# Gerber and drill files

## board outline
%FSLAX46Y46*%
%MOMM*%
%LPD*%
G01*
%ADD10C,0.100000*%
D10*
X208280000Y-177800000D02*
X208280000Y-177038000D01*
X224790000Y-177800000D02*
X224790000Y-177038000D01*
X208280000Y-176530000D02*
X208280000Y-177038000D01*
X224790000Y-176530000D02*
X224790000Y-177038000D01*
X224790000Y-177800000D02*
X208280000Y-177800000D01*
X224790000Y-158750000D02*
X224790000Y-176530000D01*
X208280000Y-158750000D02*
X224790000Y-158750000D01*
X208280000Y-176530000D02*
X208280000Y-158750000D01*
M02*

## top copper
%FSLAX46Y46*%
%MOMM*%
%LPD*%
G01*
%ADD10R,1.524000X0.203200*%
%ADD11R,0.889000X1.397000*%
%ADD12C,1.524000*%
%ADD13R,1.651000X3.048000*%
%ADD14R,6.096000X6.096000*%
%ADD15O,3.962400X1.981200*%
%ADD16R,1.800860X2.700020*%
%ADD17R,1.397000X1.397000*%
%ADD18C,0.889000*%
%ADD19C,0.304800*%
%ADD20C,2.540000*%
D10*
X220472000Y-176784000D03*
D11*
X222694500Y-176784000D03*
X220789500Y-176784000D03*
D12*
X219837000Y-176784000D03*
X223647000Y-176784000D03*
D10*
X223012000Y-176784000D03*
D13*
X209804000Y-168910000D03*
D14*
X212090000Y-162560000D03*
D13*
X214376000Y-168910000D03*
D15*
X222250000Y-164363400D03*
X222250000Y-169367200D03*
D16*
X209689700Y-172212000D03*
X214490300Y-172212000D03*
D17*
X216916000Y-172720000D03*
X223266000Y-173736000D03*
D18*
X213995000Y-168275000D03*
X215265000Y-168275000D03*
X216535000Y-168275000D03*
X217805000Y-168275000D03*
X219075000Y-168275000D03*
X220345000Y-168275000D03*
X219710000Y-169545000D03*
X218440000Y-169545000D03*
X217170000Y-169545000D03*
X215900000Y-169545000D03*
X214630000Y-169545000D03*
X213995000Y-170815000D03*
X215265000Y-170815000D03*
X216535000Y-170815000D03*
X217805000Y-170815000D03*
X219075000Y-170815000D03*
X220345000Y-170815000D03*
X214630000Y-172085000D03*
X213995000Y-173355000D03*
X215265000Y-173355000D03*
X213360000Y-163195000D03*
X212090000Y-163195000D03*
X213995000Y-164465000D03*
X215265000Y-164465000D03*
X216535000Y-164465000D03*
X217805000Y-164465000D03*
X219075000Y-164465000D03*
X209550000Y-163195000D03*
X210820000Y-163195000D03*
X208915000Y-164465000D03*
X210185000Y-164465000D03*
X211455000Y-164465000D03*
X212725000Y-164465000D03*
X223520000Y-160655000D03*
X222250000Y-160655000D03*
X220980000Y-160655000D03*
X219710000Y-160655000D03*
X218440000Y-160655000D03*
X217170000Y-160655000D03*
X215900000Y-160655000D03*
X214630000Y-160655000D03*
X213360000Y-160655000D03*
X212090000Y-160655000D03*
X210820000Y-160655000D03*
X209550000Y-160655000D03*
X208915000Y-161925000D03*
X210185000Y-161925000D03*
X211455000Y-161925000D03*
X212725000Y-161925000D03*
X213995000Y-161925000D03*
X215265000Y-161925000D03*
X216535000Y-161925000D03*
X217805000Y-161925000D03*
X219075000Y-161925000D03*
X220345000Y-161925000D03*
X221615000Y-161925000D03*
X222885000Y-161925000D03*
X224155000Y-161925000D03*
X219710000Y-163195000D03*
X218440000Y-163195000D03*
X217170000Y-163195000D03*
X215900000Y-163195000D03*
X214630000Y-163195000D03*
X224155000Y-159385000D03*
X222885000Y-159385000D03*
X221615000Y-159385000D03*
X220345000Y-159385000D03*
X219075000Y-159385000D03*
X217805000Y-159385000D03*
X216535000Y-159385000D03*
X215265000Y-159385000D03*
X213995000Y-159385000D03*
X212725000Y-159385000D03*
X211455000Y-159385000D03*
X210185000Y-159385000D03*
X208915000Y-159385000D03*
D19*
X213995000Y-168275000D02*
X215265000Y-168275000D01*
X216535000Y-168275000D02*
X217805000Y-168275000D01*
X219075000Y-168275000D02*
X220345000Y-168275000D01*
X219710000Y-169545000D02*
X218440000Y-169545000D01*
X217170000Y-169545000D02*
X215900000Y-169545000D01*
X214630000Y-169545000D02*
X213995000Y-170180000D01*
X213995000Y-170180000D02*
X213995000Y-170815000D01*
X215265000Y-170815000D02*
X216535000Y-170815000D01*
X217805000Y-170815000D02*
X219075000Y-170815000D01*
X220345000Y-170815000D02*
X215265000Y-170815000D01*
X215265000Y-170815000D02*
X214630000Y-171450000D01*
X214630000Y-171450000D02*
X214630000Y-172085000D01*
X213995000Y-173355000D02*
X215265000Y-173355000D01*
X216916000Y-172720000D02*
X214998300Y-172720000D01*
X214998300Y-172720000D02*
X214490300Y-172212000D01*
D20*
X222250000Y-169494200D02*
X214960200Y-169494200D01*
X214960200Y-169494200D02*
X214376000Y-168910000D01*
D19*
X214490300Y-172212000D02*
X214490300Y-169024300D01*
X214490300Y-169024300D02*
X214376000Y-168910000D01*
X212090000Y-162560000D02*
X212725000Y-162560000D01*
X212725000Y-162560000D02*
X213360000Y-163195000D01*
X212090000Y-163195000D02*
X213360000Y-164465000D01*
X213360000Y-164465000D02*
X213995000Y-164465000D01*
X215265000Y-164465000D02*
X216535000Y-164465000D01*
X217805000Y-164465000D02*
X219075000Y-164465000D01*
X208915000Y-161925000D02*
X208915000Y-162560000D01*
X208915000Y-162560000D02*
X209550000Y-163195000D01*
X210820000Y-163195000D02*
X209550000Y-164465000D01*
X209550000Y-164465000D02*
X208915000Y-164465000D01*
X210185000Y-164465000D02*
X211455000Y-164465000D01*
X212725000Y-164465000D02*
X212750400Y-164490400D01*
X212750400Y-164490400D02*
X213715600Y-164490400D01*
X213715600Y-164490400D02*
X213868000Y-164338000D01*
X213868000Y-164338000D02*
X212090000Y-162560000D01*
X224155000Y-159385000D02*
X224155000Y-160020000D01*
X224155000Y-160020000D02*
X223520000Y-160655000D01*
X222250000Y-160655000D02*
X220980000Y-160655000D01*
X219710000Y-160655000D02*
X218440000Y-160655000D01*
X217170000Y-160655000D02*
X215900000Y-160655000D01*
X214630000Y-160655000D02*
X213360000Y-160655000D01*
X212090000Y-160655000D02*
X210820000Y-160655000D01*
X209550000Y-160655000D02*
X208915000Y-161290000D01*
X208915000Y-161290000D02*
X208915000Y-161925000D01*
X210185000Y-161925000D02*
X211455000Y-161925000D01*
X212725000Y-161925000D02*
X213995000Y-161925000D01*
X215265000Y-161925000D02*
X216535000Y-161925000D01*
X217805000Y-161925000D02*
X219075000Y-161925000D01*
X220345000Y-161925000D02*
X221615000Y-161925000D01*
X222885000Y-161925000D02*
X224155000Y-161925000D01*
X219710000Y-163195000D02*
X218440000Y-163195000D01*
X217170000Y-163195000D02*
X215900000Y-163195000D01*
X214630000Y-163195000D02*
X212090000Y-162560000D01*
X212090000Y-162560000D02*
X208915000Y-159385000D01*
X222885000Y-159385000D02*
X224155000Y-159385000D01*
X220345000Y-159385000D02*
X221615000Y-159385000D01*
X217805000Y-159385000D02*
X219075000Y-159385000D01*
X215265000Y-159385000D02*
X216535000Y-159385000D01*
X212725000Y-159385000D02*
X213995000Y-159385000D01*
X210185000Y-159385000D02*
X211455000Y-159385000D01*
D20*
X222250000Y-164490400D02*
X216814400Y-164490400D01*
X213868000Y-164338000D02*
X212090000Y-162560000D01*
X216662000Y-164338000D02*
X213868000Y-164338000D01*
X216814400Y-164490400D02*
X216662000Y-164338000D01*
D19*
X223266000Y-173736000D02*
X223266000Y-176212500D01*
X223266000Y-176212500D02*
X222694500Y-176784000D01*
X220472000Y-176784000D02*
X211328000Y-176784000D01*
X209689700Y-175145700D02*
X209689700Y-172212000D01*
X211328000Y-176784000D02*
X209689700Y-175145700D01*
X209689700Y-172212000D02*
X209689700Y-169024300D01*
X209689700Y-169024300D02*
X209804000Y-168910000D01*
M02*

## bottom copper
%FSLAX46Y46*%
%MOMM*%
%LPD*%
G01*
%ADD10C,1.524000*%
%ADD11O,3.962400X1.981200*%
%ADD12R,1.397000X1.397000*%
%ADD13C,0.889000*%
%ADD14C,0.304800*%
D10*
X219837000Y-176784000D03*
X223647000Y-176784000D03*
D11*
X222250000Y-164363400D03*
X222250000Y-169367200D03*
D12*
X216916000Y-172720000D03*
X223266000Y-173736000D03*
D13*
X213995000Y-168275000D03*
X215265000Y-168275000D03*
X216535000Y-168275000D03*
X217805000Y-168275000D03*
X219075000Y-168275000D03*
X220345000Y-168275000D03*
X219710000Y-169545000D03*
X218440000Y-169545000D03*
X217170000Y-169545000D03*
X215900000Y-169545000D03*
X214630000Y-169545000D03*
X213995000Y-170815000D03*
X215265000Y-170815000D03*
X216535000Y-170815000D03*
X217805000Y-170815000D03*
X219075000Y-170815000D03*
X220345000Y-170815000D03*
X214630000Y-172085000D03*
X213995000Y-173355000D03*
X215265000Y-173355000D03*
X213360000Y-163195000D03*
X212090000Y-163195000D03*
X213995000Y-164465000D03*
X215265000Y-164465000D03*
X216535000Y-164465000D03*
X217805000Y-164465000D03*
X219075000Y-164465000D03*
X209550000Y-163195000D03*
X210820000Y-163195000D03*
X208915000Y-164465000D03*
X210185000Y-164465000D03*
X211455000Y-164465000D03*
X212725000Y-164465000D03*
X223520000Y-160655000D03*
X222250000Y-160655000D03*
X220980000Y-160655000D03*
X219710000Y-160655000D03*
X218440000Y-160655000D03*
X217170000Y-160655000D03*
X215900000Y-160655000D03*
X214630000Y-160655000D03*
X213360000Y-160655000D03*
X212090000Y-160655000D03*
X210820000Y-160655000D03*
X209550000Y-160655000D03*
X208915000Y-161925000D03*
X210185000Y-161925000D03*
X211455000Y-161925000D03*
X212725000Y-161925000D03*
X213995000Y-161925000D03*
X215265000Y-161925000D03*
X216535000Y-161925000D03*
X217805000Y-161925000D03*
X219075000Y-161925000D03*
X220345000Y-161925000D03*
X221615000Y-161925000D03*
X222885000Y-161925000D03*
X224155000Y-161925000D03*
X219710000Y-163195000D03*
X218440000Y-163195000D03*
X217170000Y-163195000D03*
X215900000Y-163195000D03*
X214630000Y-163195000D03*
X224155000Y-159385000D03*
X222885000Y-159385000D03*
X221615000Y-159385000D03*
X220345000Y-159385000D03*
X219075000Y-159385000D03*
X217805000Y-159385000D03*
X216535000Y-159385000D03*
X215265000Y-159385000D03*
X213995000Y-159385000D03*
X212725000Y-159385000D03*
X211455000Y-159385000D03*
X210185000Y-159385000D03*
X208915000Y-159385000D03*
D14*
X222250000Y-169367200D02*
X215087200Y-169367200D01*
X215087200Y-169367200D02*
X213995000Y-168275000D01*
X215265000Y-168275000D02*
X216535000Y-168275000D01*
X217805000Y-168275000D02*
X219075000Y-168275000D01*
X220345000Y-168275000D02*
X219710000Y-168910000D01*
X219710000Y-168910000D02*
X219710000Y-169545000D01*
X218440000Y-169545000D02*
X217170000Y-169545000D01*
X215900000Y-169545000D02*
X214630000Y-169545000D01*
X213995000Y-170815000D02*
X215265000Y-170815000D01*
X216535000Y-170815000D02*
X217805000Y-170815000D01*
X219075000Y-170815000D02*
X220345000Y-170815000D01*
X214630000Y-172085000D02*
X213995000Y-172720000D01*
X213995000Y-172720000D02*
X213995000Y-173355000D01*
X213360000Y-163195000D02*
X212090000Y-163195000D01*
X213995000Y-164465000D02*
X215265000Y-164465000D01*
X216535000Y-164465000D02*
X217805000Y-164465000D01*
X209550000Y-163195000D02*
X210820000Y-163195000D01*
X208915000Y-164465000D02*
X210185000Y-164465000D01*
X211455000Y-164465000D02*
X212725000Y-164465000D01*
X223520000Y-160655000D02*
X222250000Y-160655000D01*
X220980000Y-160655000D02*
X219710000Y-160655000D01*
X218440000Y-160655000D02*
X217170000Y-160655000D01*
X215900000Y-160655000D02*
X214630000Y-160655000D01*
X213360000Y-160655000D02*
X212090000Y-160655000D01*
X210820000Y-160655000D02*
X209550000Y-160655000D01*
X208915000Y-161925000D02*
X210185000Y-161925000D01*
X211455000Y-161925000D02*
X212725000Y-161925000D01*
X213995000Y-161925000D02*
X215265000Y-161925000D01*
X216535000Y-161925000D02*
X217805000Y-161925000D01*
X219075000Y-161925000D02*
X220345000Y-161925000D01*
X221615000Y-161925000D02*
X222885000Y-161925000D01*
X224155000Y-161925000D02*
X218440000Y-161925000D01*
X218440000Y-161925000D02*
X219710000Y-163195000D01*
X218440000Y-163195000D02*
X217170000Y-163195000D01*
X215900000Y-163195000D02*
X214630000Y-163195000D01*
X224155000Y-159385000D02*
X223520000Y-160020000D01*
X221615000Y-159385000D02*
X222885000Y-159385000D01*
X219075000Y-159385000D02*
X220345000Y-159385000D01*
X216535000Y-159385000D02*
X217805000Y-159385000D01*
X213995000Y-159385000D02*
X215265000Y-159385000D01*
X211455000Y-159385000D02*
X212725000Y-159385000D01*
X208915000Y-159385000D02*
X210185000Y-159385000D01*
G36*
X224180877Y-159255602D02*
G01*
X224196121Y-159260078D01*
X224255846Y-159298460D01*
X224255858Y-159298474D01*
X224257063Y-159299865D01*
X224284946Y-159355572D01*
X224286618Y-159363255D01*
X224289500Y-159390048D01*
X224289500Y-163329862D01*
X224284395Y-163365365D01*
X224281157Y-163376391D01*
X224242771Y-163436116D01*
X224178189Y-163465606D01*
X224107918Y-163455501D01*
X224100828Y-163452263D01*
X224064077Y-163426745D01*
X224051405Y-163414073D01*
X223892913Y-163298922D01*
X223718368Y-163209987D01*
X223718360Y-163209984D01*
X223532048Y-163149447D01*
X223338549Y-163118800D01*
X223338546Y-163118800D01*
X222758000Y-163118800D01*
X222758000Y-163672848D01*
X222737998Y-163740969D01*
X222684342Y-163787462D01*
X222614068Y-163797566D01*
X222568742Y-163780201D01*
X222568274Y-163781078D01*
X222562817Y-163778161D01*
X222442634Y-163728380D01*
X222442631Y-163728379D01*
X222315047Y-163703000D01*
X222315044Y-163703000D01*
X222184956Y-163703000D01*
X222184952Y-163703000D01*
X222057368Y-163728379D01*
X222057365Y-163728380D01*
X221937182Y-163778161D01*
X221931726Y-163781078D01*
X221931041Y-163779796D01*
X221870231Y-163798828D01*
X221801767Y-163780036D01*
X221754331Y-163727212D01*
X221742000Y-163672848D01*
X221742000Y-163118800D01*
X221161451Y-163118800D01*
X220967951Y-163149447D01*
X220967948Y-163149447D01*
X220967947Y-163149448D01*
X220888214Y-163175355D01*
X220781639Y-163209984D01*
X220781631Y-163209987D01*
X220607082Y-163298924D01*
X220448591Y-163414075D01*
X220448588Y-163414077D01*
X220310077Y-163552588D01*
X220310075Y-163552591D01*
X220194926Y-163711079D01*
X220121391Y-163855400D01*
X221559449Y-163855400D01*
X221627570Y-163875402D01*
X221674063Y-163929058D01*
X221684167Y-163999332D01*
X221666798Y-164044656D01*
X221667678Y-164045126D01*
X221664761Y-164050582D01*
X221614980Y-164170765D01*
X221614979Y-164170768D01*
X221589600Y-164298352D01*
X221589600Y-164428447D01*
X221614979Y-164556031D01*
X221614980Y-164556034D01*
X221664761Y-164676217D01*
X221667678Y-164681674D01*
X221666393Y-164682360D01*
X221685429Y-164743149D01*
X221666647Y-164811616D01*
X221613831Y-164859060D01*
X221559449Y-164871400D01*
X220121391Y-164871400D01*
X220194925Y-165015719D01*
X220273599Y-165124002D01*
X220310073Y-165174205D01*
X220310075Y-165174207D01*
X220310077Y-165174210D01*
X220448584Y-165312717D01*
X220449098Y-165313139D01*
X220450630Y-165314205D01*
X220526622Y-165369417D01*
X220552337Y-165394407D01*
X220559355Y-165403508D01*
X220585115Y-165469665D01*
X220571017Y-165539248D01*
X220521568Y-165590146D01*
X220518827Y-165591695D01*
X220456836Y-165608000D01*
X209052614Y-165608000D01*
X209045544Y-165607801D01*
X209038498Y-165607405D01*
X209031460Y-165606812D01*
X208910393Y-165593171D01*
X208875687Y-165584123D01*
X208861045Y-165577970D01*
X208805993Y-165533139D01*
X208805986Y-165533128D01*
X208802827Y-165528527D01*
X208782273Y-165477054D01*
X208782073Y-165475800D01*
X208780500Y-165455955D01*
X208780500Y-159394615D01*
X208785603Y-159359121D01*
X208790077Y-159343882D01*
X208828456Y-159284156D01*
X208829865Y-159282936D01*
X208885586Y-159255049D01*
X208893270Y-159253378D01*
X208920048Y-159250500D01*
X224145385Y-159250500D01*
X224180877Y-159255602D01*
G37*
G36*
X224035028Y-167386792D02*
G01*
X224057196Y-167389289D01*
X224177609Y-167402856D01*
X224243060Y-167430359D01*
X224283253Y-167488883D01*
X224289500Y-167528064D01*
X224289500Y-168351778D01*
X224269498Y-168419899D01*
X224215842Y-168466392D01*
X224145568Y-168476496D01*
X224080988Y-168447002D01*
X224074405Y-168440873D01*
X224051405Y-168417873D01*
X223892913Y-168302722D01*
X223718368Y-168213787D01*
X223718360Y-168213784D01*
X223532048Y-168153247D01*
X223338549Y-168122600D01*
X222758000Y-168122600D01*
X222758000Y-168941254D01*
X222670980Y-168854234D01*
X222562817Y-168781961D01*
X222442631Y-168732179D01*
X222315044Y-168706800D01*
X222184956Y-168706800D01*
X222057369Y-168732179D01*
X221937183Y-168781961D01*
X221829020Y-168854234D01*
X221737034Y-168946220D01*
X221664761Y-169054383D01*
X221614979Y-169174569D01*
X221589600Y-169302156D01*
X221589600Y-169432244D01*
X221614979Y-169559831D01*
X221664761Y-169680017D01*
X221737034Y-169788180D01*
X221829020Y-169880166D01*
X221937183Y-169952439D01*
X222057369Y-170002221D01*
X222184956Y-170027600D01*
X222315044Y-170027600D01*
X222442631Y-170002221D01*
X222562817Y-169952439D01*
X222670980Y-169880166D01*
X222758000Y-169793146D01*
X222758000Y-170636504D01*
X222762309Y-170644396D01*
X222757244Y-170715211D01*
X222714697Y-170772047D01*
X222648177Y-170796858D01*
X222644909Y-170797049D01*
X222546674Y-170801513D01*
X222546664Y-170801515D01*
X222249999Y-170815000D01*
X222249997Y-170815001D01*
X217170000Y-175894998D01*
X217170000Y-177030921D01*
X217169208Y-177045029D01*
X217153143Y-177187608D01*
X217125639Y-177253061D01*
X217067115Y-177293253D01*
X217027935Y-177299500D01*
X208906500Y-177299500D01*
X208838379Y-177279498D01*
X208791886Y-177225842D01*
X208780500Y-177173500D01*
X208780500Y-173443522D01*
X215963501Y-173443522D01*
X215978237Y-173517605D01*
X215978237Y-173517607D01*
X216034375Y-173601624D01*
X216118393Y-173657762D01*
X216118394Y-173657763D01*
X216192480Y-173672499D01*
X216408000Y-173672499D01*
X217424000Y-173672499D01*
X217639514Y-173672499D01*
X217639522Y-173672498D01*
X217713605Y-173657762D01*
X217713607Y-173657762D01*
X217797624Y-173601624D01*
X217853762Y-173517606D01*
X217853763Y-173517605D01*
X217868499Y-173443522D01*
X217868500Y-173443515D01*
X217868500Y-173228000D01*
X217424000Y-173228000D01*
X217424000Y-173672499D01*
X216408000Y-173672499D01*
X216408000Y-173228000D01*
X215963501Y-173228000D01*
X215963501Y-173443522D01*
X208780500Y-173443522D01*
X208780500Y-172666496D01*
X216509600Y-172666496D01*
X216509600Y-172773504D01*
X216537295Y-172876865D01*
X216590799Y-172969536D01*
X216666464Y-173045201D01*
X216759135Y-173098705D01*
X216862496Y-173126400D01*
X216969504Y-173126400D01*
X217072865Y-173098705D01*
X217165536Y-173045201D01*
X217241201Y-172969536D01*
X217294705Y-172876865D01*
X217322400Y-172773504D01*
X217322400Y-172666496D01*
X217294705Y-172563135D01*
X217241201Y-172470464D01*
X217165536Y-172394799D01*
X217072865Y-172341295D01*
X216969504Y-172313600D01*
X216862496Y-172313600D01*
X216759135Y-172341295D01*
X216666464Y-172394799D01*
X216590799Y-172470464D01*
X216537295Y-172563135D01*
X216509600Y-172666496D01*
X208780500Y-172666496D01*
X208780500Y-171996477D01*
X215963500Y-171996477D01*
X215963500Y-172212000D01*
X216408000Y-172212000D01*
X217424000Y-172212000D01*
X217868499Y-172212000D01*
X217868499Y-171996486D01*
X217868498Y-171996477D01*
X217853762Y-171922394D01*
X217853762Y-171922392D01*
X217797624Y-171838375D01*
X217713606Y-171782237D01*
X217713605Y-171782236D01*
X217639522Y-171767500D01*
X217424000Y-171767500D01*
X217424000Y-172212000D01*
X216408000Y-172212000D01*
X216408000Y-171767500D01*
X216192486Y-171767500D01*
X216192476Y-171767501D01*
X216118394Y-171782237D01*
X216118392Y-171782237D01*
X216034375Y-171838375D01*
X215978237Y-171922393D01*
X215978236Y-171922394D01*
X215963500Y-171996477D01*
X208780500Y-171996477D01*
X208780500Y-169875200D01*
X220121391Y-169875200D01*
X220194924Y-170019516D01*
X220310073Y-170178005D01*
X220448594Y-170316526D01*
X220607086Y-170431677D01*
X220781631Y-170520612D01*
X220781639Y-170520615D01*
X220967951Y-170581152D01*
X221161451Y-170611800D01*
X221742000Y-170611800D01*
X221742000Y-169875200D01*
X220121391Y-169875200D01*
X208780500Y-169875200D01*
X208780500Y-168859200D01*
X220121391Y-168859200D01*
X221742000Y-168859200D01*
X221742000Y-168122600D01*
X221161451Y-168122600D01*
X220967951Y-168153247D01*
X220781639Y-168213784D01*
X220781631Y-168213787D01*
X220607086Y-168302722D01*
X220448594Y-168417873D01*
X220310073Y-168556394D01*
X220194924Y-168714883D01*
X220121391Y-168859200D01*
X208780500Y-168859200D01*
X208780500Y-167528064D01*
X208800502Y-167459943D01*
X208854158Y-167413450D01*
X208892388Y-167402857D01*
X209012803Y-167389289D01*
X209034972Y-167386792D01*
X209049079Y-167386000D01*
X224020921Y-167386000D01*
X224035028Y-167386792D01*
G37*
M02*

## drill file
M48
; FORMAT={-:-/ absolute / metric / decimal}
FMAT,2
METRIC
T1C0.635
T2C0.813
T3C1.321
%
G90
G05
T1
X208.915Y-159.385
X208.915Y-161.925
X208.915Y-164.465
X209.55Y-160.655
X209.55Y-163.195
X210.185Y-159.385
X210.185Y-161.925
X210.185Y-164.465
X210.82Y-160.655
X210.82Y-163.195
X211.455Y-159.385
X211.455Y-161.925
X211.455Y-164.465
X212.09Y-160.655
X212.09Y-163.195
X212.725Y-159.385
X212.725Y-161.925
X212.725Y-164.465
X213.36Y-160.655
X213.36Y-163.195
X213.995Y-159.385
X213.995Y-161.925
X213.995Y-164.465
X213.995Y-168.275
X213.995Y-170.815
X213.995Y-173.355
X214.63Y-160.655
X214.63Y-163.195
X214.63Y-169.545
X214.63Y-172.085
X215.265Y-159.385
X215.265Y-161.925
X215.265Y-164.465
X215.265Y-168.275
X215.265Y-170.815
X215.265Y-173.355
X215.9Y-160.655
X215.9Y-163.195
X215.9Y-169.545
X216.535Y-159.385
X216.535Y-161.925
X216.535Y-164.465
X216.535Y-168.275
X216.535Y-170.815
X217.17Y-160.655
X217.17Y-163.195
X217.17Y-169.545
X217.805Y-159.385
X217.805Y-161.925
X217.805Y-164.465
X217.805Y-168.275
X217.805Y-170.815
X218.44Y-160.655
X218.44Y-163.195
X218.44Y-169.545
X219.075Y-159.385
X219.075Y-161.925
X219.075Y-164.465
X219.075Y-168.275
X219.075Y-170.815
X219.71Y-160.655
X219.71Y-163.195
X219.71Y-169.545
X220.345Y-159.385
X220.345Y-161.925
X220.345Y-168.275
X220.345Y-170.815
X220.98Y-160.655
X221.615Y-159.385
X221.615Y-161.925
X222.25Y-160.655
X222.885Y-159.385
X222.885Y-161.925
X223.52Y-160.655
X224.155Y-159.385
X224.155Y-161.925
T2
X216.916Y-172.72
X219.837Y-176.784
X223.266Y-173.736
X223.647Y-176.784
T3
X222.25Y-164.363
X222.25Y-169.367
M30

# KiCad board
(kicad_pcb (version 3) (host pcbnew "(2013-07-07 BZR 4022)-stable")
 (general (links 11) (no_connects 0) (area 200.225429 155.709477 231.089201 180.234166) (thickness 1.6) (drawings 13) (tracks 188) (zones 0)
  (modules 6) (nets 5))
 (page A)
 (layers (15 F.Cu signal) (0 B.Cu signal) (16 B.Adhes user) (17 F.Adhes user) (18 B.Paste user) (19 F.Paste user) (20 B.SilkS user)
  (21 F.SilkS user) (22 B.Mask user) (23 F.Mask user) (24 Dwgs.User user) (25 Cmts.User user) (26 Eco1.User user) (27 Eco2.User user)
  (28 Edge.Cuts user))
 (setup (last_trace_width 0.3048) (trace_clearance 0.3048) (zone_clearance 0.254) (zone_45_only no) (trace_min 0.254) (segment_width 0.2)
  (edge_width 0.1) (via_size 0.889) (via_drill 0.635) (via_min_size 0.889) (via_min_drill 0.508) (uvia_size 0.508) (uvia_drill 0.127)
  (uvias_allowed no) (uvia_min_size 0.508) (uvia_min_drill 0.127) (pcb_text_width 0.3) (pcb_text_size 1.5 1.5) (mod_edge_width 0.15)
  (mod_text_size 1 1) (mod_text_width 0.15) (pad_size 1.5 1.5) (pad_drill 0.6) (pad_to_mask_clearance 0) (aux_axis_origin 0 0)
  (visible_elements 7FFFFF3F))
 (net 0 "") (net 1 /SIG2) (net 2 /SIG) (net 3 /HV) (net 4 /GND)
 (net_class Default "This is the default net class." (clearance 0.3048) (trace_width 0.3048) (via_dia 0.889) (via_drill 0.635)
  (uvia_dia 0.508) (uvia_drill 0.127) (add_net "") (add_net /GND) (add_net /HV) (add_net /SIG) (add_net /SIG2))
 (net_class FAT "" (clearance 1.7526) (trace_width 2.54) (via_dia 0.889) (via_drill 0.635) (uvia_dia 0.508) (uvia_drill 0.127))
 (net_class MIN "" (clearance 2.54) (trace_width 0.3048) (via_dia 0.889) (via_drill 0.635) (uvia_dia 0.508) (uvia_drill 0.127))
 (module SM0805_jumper (layer F.Cu) (at 221.742 176.784 180)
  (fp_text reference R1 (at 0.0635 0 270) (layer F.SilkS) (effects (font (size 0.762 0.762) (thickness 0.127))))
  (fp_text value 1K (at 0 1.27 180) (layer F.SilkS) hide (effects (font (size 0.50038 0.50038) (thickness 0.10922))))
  (pad 2 smd rect (at 1.27 0 180) (size 1.524 0.2032) (layers F.Cu F.Paste F.Mask) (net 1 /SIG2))
  (pad 1 smd rect (at -0.9525 0 180) (size 0.889 1.397) (layers F.Cu F.Paste F.Mask) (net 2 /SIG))
  (pad 2 smd rect (at 0.9525 0 180) (size 0.889 1.397) (layers F.Cu F.Paste F.Mask) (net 1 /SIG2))
  (pad 2 thru_hole circle (at 1.905 0 180) (size 1.524 1.524) (drill 0.8128) (layers *.Cu *.Mask F.SilkS) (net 1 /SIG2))
  (pad 1 thru_hole circle (at -1.905 0 180) (size 1.524 1.524) (drill 0.8128) (layers *.Cu *.Mask F.SilkS) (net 2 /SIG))
  (pad 1 smd rect (at -1.27 0 180) (size 1.524 0.2032) (layers F.Cu F.Paste F.Mask) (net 2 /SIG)))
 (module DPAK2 (layer F.Cu) (at 212.09 168.91)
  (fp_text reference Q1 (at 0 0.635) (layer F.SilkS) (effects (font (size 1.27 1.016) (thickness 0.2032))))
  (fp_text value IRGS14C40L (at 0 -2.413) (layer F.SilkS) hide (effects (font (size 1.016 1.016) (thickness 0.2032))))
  (pad 1 smd rect (at -2.286 0) (size 1.651 3.048) (layers F.Cu F.Paste F.Mask) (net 1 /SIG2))
  (pad 2 smd rect (at 0 -6.35) (size 6.096 6.096) (layers F.Cu F.Paste F.Mask) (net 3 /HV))
  (pad 3 smd rect (at 2.286 0) (size 1.651 3.048) (layers F.Cu F.Paste F.Mask) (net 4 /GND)))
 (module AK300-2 (layer F.Cu) (at 222.25 166.878 270)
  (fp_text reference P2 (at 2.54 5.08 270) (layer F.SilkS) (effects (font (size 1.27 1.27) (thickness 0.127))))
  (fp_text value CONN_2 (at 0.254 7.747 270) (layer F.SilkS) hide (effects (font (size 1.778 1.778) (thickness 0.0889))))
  (pad 1 thru_hole oval (at -2.5146 0 270) (size 1.9812 3.9624) (drill 1.3208) (layers *.Cu F.Paste F.SilkS F.Mask) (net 3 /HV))
  (pad 2 thru_hole oval (at 2.4892 0 270) (size 1.9812 3.9624) (drill 1.3208) (layers *.Cu F.Paste F.SilkS F.Mask) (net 4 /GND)))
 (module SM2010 (layer F.Cu) (at 212.09 172.212)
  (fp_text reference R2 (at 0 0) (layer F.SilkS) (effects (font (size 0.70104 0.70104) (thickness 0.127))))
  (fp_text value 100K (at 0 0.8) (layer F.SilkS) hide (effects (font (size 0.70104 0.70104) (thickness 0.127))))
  (pad 1 smd rect (at -2.4003 0) (size 1.80086 2.70002) (layers F.Cu F.Paste F.Mask) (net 1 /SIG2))
  (pad 2 smd rect (at 2.4003 0) (size 1.80086 2.70002) (layers F.Cu F.Paste F.Mask) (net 4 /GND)))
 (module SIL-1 (layer F.Cu) (at 216.916 172.72)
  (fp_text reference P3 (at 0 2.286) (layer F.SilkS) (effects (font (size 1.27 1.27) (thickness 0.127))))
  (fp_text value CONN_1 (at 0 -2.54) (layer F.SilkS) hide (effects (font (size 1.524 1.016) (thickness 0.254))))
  (pad 1 thru_hole rect (at 0 0) (size 1.397 1.397) (drill 0.8128) (layers *.Cu *.Mask F.SilkS) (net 4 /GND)))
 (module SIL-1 (layer F.Cu) (at 223.266 173.736 180)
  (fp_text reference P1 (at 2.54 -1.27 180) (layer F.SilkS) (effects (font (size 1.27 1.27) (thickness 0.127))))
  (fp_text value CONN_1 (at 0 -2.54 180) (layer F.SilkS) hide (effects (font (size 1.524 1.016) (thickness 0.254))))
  (pad 1 thru_hole rect (at 0 0 180) (size 1.397 1.397) (drill 0.8128) (layers *.Cu *.Mask F.SilkS) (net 2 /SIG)))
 (gr_line (start 208.28 177.8) (end 208.28 177.038) (angle 90) (layer Edge.Cuts) (width 0.1))
 (gr_line (start 224.79 177.8) (end 224.79 177.038) (angle 90) (layer Edge.Cuts) (width 0.1))
 (gr_line (start 208.28 176.53) (end 208.28 177.038) (angle 90) (layer Edge.Cuts) (width 0.1))
 (gr_line (start 224.79 176.53) (end 224.79 177.038) (angle 90) (layer Edge.Cuts) (width 0.1))
 (gr_line (start 224.79 177.8) (end 208.28 177.8) (angle 90) (layer Edge.Cuts) (width 0.1))
 (gr_line (start 224.79 158.75) (end 224.79 176.53) (angle 90) (layer Edge.Cuts) (width 0.1))
 (gr_line (start 208.28 158.75) (end 224.79 158.75) (angle 90) (layer Edge.Cuts) (width 0.1))
 (gr_line (start 208.28 176.53) (end 208.28 158.75) (angle 90) (layer Edge.Cuts) (width 0.1))
 (segment (start 222.25 169.3672) (end 215.0872 169.3672) (width 0.3048) (layer B.Cu) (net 4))
 (segment (start 215.0872 169.3672) (end 213.995 168.275) (width 0.3048) (layer B.Cu) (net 4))
 (via (at 213.995 168.275) (size 0.889) (layers F.Cu B.Cu) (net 4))
 (segment (start 213.995 168.275) (end 215.265 168.275) (width 0.3048) (layer F.Cu) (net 4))
 (via (at 215.265 168.275) (size 0.889) (layers F.Cu B.Cu) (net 4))
 (segment (start 215.265 168.275) (end 216.535 168.275) (width 0.3048) (layer B.Cu) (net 4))
 (via (at 216.535 168.275) (size 0.889) (layers F.Cu B.Cu) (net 4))
 (segment (start 216.535 168.275) (end 217.805 168.275) (width 0.3048) (layer F.Cu) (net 4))
 (via (at 217.805 168.275) (size 0.889) (layers F.Cu B.Cu) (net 4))
 (segment (start 217.805 168.275) (end 219.075 168.275) (width 0.3048) (layer B.Cu) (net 4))
 (via (at 219.075 168.275) (size 0.889) (layers F.Cu B.Cu) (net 4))
 (segment (start 219.075 168.275) (end 220.345 168.275) (width 0.3048) (layer F.Cu) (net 4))
 (via (at 220.345 168.275) (size 0.889) (layers F.Cu B.Cu) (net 4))
 (segment (start 220.345 168.275) (end 219.71 168.91) (width 0.3048) (layer B.Cu) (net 4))
 (segment (start 219.71 168.91) (end 219.71 169.545) (width 0.3048) (layer B.Cu) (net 4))
 (via (at 219.71 169.545) (size 0.889) (layers F.Cu B.Cu) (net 4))
 (segment (start 219.71 169.545) (end 218.44 169.545) (width 0.3048) (layer F.Cu) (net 4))
 (via (at 218.44 169.545) (size 0.889) (layers F.Cu B.Cu) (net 4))
 (segment (start 218.44 169.545) (end 217.17 169.545) (width 0.3048) (layer B.Cu) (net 4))
 (via (at 217.17 169.545) (size 0.889) (layers F.Cu B.Cu) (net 4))
 (segment (start 217.17 169.545) (end 215.9 169.545) (width 0.3048) (layer F.Cu) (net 4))
 (via (at 215.9 169.545) (size 0.889) (layers F.Cu B.Cu) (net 4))
 (segment (start 215.9 169.545) (end 214.63 169.545) (width 0.3048) (layer B.Cu) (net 4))
 (via (at 214.63 169.545) (size 0.889) (layers F.Cu B.Cu) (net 4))
 (segment (start 214.63 169.545) (end 213.995 170.18) (width 0.3048) (layer F.Cu) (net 4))
 (segment (start 213.995 170.18) (end 213.995 170.815) (width 0.3048) (layer F.Cu) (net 4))
 (via (at 213.995 170.815) (size 0.889) (layers F.Cu B.Cu) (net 4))
 (segment (start 213.995 170.815) (end 215.265 170.815) (width 0.3048) (layer B.Cu) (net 4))
 (via (at 215.265 170.815) (size 0.889) (layers F.Cu B.Cu) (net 4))
 (segment (start 215.265 170.815) (end 216.535 170.815) (width 0.3048) (layer F.Cu) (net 4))
 (via (at 216.535 170.815) (size 0.889) (layers F.Cu B.Cu) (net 4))
 (segment (start 216.535 170.815) (end 217.805 170.815) (width 0.3048) (layer B.Cu) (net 4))
 (via (at 217.805 170.815) (size 0.889) (layers F.Cu B.Cu) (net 4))
 (segment (start 217.805 170.815) (end 219.075 170.815) (width 0.3048) (layer F.Cu) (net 4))
 (via (at 219.075 170.815) (size 0.889) (layers F.Cu B.Cu) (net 4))
 (segment (start 219.075 170.815) (end 220.345 170.815) (width 0.3048) (layer B.Cu) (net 4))
 (via (at 220.345 170.815) (size 0.889) (layers F.Cu B.Cu) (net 4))
 (segment (start 220.345 170.815) (end 215.265 170.815) (width 0.3048) (layer F.Cu) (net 4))
 (segment (start 215.265 170.815) (end 214.63 171.45) (width 0.3048) (layer F.Cu) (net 4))
 (segment (start 214.63 171.45) (end 214.63 172.085) (width 0.3048) (layer F.Cu) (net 4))
 (via (at 214.63 172.085) (size 0.889) (layers F.Cu B.Cu) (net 4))
 (segment (start 214.63 172.085) (end 213.995 172.72) (width 0.3048) (layer B.Cu) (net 4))
 (segment (start 213.995 172.72) (end 213.995 173.355) (width 0.3048) (layer B.Cu) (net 4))
 (via (at 213.995 173.355) (size 0.889) (layers F.Cu B.Cu) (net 4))
 (segment (start 213.995 173.355) (end 215.265 173.355) (width 0.3048) (layer F.Cu) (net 4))
 (via (at 215.265 173.355) (size 0.889) (layers F.Cu B.Cu) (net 4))
 (segment (start 216.916 172.72) (end 214.9983 172.72) (width 0.3048) (layer F.Cu) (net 4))
 (segment (start 214.9983 172.72) (end 214.4903 172.212) (width 0.3048) (layer F.Cu) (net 4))
 (segment (start 222.25 169.4942) (end 214.9602 169.4942) (width 2.54) (layer F.Cu) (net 4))
 (segment (start 214.9602 169.4942) (end 214.376 168.91) (width 2.54) (layer F.Cu) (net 4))
 (segment (start 214.4903 172.212) (end 214.4903 169.0243) (width 0.3048) (layer F.Cu) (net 4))
 (segment (start 214.4903 169.0243) (end 214.376 168.91) (width 0.3048) (layer F.Cu) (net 4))
 (segment (start 212.09 162.56) (end 212.725 162.56) (width 0.3048) (layer F.Cu) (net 3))
 (segment (start 212.725 162.56) (end 213.36 163.195) (width 0.3048) (layer F.Cu) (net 3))
 (via (at 213.36 163.195) (size 0.889) (layers F.Cu B.Cu) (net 3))
 (segment (start 213.36 163.195) (end 212.09 163.195) (width 0.3048) (layer B.Cu) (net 3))
 (via (at 212.09 163.195) (size 0.889) (layers F.Cu B.Cu) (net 3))
 (segment (start 212.09 163.195) (end 213.36 164.465) (width 0.3048) (layer F.Cu) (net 3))
 (segment (start 213.36 164.465) (end 213.995 164.465) (width 0.3048) (layer F.Cu) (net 3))
 (via (at 213.995 164.465) (size 0.889) (layers F.Cu B.Cu) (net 3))
 (segment (start 213.995 164.465) (end 215.265 164.465) (width 0.3048) (layer B.Cu) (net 3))
 (via (at 215.265 164.465) (size 0.889) (layers F.Cu B.Cu) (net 3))
 (segment (start 215.265 164.465) (end 216.535 164.465) (width 0.3048) (layer F.Cu) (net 3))
 (via (at 216.535 164.465) (size 0.889) (layers F.Cu B.Cu) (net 3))
 (segment (start 216.535 164.465) (end 217.805 164.465) (width 0.3048) (layer B.Cu) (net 3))
 (via (at 217.805 164.465) (size 0.889) (layers F.Cu B.Cu) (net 3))
 (segment (start 217.805 164.465) (end 219.075 164.465) (width 0.3048) (layer F.Cu) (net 3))
 (via (at 219.075 164.465) (size 0.889) (layers F.Cu B.Cu) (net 3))
 (segment (start 208.915 161.925) (end 208.915 162.56) (width 0.3048) (layer F.Cu) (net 3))
 (segment (start 208.915 162.56) (end 209.55 163.195) (width 0.3048) (layer F.Cu) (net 3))
 (via (at 209.55 163.195) (size 0.889) (layers F.Cu B.Cu) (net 3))
 (segment (start 209.55 163.195) (end 210.82 163.195) (width 0.3048) (layer B.Cu) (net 3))
 (via (at 210.82 163.195) (size 0.889) (layers F.Cu B.Cu) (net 3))
 (segment (start 210.82 163.195) (end 209.55 164.465) (width 0.3048) (layer F.Cu) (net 3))
 (segment (start 209.55 164.465) (end 208.915 164.465) (width 0.3048) (layer F.Cu) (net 3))
 (via (at 208.915 164.465) (size 0.889) (layers F.Cu B.Cu) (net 3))
 (segment (start 208.915 164.465) (end 210.185 164.465) (width 0.3048) (layer B.Cu) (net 3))
 (via (at 210.185 164.465) (size 0.889) (layers F.Cu B.Cu) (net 3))
 (segment (start 210.185 164.465) (end 211.455 164.465) (width 0.3048) (layer F.Cu) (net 3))
 (via (at 211.455 164.465) (size 0.889) (layers F.Cu B.Cu) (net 3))
 (segment (start 211.455 164.465) (end 212.725 164.465) (width 0.3048) (layer B.Cu) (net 3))
 (via (at 212.725 164.465) (size 0.889) (layers F.Cu B.Cu) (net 3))
 (segment (start 212.725 164.465) (end 212.7504 164.4904) (width 0.3048) (layer F.Cu) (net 3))
 (segment (start 212.7504 164.4904) (end 213.7156 164.4904) (width 0.3048) (layer F.Cu) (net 3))
 (segment (start 213.7156 164.4904) (end 213.868 164.338) (width 0.3048) (layer F.Cu) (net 3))
 (segment (start 213.868 164.338) (end 212.09 162.56) (width 0.3048) (layer F.Cu) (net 3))
 (segment (start 224.155 159.385) (end 224.155 160.02) (width 0.3048) (layer F.Cu) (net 3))
 (segment (start 224.155 160.02) (end 223.52 160.655) (width 0.3048) (layer F.Cu) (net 3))
 (via (at 223.52 160.655) (size 0.889) (layers F.Cu B.Cu) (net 3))
 (segment (start 223.52 160.655) (end 222.25 160.655) (width 0.3048) (layer B.Cu) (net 3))
 (via (at 222.25 160.655) (size 0.889) (layers F.Cu B.Cu) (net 3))
 (segment (start 222.25 160.655) (end 220.98 160.655) (width 0.3048) (layer F.Cu) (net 3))
 (via (at 220.98 160.655) (size 0.889) (layers F.Cu B.Cu) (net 3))
 (segment (start 220.98 160.655) (end 219.71 160.655) (width 0.3048) (layer B.Cu) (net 3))
 (via (at 219.71 160.655) (size 0.889) (layers F.Cu B.Cu) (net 3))
 (segment (start 219.71 160.655) (end 218.44 160.655) (width 0.3048) (layer F.Cu) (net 3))
 (via (at 218.44 160.655) (size 0.889) (layers F.Cu B.Cu) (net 3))
 (segment (start 218.44 160.655) (end 217.17 160.655) (width 0.3048) (layer B.Cu) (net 3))
 (via (at 217.17 160.655) (size 0.889) (layers F.Cu B.Cu) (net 3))
 (segment (start 217.17 160.655) (end 215.9 160.655) (width 0.3048) (layer F.Cu) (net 3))
 (via (at 215.9 160.655) (size 0.889) (layers F.Cu B.Cu) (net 3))
 (segment (start 215.9 160.655) (end 214.63 160.655) (width 0.3048) (layer B.Cu) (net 3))
 (via (at 214.63 160.655) (size 0.889) (layers F.Cu B.Cu) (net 3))
 (segment (start 214.63 160.655) (end 213.36 160.655) (width 0.3048) (layer F.Cu) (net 3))
 (via (at 213.36 160.655) (size 0.889) (layers F.Cu B.Cu) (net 3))
 (segment (start 213.36 160.655) (end 212.09 160.655) (width 0.3048) (layer B.Cu) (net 3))
 (via (at 212.09 160.655) (size 0.889) (layers F.Cu B.Cu) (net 3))
 (segment (start 212.09 160.655) (end 210.82 160.655) (width 0.3048) (layer F.Cu) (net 3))
 (via (at 210.82 160.655) (size 0.889) (layers F.Cu B.Cu) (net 3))
 (segment (start 210.82 160.655) (end 209.55 160.655) (width 0.3048) (layer B.Cu) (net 3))
 (via (at 209.55 160.655) (size 0.889) (layers F.Cu B.Cu) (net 3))
 (segment (start 209.55 160.655) (end 208.915 161.29) (width 0.3048) (layer F.Cu) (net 3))
 (segment (start 208.915 161.29) (end 208.915 161.925) (width 0.3048) (layer F.Cu) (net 3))
 (via (at 208.915 161.925) (size 0.889) (layers F.Cu B.Cu) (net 3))
 (segment (start 208.915 161.925) (end 210.185 161.925) (width 0.3048) (layer B.Cu) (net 3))
 (via (at 210.185 161.925) (size 0.889) (layers F.Cu B.Cu) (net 3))
 (segment (start 210.185 161.925) (end 211.455 161.925) (width 0.3048) (layer F.Cu) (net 3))
 (via (at 211.455 161.925) (size 0.889) (layers F.Cu B.Cu) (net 3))
 (segment (start 211.455 161.925) (end 212.725 161.925) (width 0.3048) (layer B.Cu) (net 3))
 (via (at 212.725 161.925) (size 0.889) (layers F.Cu B.Cu) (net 3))
 (segment (start 212.725 161.925) (end 213.995 161.925) (width 0.3048) (layer F.Cu) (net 3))
 (via (at 213.995 161.925) (size 0.889) (layers F.Cu B.Cu) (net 3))
 (segment (start 213.995 161.925) (end 215.265 161.925) (width 0.3048) (layer B.Cu) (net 3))
 (via (at 215.265 161.925) (size 0.889) (layers F.Cu B.Cu) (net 3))
 (segment (start 215.265 161.925) (end 216.535 161.925) (width 0.3048) (layer F.Cu) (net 3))
 (via (at 216.535 161.925) (size 0.889) (layers F.Cu B.Cu) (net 3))
 (segment (start 216.535 161.925) (end 217.805 161.925) (width 0.3048) (layer B.Cu) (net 3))
 (via (at 217.805 161.925) (size 0.889) (layers F.Cu B.Cu) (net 3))
 (segment (start 217.805 161.925) (end 219.075 161.925) (width 0.3048) (layer F.Cu) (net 3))
 (via (at 219.075 161.925) (size 0.889) (layers F.Cu B.Cu) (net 3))
 (segment (start 219.075 161.925) (end 220.345 161.925) (width 0.3048) (layer B.Cu) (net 3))
 (via (at 220.345 161.925) (size 0.889) (layers F.Cu B.Cu) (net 3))
 (segment (start 220.345 161.925) (end 221.615 161.925) (width 0.3048) (layer F.Cu) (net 3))
 (via (at 221.615 161.925) (size 0.889) (layers F.Cu B.Cu) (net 3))
 (segment (start 221.615 161.925) (end 222.885 161.925) (width 0.3048) (layer B.Cu) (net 3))
 (via (at 222.885 161.925) (size 0.889) (layers F.Cu B.Cu) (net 3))
 (segment (start 222.885 161.925) (end 224.155 161.925) (width 0.3048) (layer F.Cu) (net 3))
 (via (at 224.155 161.925) (size 0.889) (layers F.Cu B.Cu) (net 3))
 (segment (start 224.155 161.925) (end 218.44 161.925) (width 0.3048) (layer B.Cu) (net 3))
 (segment (start 218.44 161.925) (end 219.71 163.195) (width 0.3048) (layer B.Cu) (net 3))
 (via (at 219.71 163.195) (size 0.889) (layers F.Cu B.Cu) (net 3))
 (segment (start 219.71 163.195) (end 218.44 163.195) (width 0.3048) (layer F.Cu) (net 3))
 (via (at 218.44 163.195) (size 0.889) (layers F.Cu B.Cu) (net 3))
 (segment (start 218.44 163.195) (end 217.17 163.195) (width 0.3048) (layer B.Cu) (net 3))
 (via (at 217.17 163.195) (size 0.889) (layers F.Cu B.Cu) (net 3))
 (segment (start 217.17 163.195) (end 215.9 163.195) (width 0.3048) (layer F.Cu) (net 3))
 (via (at 215.9 163.195) (size 0.889) (layers F.Cu B.Cu) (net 3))
 (segment (start 215.9 163.195) (end 214.63 163.195) (width 0.3048) (layer B.Cu) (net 3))
 (via (at 214.63 163.195) (size 0.889) (layers F.Cu B.Cu) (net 3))
 (segment (start 214.63 163.195) (end 212.09 162.56) (width 0.3048) (layer F.Cu) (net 3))
 (segment (start 212.09 162.56) (end 208.915 159.385) (width 0.3048) (layer F.Cu) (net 3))
 (segment (start 224.155 159.385) (end 223.52 160.02) (width 0.3048) (layer B.Cu) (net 3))
 (via (at 224.155 159.385) (size 0.889) (layers F.Cu B.Cu) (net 3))
 (segment (start 222.885 159.385) (end 224.155 159.385) (width 0.3048) (layer F.Cu) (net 3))
 (via (at 222.885 159.385) (size 0.889) (layers F.Cu B.Cu) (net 3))
 (segment (start 221.615 159.385) (end 222.885 159.385) (width 0.3048) (layer B.Cu) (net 3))
 (via (at 221.615 159.385) (size 0.889) (layers F.Cu B.Cu) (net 3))
 (segment (start 220.345 159.385) (end 221.615 159.385) (width 0.3048) (layer F.Cu) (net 3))
 (via (at 220.345 159.385) (size 0.889) (layers F.Cu B.Cu) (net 3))
 (segment (start 219.075 159.385) (end 220.345 159.385) (width 0.3048) (layer B.Cu) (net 3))
 (via (at 219.075 159.385) (size 0.889) (layers F.Cu B.Cu) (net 3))
 (segment (start 217.805 159.385) (end 219.075 159.385) (width 0.3048) (layer F.Cu) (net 3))
 (via (at 217.805 159.385) (size 0.889) (layers F.Cu B.Cu) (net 3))
 (segment (start 216.535 159.385) (end 217.805 159.385) (width 0.3048) (layer B.Cu) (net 3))
 (via (at 216.535 159.385) (size 0.889) (layers F.Cu B.Cu) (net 3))
 (segment (start 215.265 159.385) (end 216.535 159.385) (width 0.3048) (layer F.Cu) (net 3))
 (via (at 215.265 159.385) (size 0.889) (layers F.Cu B.Cu) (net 3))
 (segment (start 213.995 159.385) (end 215.265 159.385) (width 0.3048) (layer B.Cu) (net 3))
 (via (at 213.995 159.385) (size 0.889) (layers F.Cu B.Cu) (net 3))
 (segment (start 212.725 159.385) (end 213.995 159.385) (width 0.3048) (layer F.Cu) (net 3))
 (via (at 212.725 159.385) (size 0.889) (layers F.Cu B.Cu) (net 3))
 (segment (start 211.455 159.385) (end 212.725 159.385) (width 0.3048) (layer B.Cu) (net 3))
 (via (at 211.455 159.385) (size 0.889) (layers F.Cu B.Cu) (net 3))
 (segment (start 210.185 159.385) (end 211.455 159.385) (width 0.3048) (layer F.Cu) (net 3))
 (via (at 210.185 159.385) (size 0.889) (layers F.Cu B.Cu) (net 3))
 (segment (start 208.915 159.385) (end 210.185 159.385) (width 0.3048) (layer B.Cu) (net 3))
 (via (at 208.915 159.385) (size 0.889) (layers F.Cu B.Cu) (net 3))
 (segment (start 222.25 164.4904) (end 216.8144 164.4904) (width 2.54) (layer F.Cu) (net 3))
 (segment (start 213.868 164.338) (end 212.09 162.56) (width 2.54) (layer F.Cu) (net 3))
 (segment (start 216.662 164.338) (end 213.868 164.338) (width 2.54) (layer F.Cu) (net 3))
 (segment (start 216.8144 164.4904) (end 216.662 164.338) (width 2.54) (layer F.Cu) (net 3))
 (segment (start 223.266 173.736) (end 223.266 176.2125) (width 0.3048) (layer F.Cu) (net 2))
 (segment (start 223.266 176.2125) (end 222.6945 176.784) (width 0.3048) (layer F.Cu) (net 2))
 (segment (start 220.472 176.784) (end 211.328 176.784) (width 0.3048) (layer F.Cu) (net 1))
 (segment (start 209.6897 175.1457) (end 209.6897 172.212) (width 0.3048) (layer F.Cu) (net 1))
 (segment (start 211.328 176.784) (end 209.6897 175.1457) (width 0.3048) (layer F.Cu) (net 1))
 (segment (start 209.6897 172.212) (end 209.6897 169.0243) (width 0.3048) (layer F.Cu) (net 1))
 (segment (start 209.6897 169.0243) (end 209.804 168.91) (width 0.3048) (layer F.Cu) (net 1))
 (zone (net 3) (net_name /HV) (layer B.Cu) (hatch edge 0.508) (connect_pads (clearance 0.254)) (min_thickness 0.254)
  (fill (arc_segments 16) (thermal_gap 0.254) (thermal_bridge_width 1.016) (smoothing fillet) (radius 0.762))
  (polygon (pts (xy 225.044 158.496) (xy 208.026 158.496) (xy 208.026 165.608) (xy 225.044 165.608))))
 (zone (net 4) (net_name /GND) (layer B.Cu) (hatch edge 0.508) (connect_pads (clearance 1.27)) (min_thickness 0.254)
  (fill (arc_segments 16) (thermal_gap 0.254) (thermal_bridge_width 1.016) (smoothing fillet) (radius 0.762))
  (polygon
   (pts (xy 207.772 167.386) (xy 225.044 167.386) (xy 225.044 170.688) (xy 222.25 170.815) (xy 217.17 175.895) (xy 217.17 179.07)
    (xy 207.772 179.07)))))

